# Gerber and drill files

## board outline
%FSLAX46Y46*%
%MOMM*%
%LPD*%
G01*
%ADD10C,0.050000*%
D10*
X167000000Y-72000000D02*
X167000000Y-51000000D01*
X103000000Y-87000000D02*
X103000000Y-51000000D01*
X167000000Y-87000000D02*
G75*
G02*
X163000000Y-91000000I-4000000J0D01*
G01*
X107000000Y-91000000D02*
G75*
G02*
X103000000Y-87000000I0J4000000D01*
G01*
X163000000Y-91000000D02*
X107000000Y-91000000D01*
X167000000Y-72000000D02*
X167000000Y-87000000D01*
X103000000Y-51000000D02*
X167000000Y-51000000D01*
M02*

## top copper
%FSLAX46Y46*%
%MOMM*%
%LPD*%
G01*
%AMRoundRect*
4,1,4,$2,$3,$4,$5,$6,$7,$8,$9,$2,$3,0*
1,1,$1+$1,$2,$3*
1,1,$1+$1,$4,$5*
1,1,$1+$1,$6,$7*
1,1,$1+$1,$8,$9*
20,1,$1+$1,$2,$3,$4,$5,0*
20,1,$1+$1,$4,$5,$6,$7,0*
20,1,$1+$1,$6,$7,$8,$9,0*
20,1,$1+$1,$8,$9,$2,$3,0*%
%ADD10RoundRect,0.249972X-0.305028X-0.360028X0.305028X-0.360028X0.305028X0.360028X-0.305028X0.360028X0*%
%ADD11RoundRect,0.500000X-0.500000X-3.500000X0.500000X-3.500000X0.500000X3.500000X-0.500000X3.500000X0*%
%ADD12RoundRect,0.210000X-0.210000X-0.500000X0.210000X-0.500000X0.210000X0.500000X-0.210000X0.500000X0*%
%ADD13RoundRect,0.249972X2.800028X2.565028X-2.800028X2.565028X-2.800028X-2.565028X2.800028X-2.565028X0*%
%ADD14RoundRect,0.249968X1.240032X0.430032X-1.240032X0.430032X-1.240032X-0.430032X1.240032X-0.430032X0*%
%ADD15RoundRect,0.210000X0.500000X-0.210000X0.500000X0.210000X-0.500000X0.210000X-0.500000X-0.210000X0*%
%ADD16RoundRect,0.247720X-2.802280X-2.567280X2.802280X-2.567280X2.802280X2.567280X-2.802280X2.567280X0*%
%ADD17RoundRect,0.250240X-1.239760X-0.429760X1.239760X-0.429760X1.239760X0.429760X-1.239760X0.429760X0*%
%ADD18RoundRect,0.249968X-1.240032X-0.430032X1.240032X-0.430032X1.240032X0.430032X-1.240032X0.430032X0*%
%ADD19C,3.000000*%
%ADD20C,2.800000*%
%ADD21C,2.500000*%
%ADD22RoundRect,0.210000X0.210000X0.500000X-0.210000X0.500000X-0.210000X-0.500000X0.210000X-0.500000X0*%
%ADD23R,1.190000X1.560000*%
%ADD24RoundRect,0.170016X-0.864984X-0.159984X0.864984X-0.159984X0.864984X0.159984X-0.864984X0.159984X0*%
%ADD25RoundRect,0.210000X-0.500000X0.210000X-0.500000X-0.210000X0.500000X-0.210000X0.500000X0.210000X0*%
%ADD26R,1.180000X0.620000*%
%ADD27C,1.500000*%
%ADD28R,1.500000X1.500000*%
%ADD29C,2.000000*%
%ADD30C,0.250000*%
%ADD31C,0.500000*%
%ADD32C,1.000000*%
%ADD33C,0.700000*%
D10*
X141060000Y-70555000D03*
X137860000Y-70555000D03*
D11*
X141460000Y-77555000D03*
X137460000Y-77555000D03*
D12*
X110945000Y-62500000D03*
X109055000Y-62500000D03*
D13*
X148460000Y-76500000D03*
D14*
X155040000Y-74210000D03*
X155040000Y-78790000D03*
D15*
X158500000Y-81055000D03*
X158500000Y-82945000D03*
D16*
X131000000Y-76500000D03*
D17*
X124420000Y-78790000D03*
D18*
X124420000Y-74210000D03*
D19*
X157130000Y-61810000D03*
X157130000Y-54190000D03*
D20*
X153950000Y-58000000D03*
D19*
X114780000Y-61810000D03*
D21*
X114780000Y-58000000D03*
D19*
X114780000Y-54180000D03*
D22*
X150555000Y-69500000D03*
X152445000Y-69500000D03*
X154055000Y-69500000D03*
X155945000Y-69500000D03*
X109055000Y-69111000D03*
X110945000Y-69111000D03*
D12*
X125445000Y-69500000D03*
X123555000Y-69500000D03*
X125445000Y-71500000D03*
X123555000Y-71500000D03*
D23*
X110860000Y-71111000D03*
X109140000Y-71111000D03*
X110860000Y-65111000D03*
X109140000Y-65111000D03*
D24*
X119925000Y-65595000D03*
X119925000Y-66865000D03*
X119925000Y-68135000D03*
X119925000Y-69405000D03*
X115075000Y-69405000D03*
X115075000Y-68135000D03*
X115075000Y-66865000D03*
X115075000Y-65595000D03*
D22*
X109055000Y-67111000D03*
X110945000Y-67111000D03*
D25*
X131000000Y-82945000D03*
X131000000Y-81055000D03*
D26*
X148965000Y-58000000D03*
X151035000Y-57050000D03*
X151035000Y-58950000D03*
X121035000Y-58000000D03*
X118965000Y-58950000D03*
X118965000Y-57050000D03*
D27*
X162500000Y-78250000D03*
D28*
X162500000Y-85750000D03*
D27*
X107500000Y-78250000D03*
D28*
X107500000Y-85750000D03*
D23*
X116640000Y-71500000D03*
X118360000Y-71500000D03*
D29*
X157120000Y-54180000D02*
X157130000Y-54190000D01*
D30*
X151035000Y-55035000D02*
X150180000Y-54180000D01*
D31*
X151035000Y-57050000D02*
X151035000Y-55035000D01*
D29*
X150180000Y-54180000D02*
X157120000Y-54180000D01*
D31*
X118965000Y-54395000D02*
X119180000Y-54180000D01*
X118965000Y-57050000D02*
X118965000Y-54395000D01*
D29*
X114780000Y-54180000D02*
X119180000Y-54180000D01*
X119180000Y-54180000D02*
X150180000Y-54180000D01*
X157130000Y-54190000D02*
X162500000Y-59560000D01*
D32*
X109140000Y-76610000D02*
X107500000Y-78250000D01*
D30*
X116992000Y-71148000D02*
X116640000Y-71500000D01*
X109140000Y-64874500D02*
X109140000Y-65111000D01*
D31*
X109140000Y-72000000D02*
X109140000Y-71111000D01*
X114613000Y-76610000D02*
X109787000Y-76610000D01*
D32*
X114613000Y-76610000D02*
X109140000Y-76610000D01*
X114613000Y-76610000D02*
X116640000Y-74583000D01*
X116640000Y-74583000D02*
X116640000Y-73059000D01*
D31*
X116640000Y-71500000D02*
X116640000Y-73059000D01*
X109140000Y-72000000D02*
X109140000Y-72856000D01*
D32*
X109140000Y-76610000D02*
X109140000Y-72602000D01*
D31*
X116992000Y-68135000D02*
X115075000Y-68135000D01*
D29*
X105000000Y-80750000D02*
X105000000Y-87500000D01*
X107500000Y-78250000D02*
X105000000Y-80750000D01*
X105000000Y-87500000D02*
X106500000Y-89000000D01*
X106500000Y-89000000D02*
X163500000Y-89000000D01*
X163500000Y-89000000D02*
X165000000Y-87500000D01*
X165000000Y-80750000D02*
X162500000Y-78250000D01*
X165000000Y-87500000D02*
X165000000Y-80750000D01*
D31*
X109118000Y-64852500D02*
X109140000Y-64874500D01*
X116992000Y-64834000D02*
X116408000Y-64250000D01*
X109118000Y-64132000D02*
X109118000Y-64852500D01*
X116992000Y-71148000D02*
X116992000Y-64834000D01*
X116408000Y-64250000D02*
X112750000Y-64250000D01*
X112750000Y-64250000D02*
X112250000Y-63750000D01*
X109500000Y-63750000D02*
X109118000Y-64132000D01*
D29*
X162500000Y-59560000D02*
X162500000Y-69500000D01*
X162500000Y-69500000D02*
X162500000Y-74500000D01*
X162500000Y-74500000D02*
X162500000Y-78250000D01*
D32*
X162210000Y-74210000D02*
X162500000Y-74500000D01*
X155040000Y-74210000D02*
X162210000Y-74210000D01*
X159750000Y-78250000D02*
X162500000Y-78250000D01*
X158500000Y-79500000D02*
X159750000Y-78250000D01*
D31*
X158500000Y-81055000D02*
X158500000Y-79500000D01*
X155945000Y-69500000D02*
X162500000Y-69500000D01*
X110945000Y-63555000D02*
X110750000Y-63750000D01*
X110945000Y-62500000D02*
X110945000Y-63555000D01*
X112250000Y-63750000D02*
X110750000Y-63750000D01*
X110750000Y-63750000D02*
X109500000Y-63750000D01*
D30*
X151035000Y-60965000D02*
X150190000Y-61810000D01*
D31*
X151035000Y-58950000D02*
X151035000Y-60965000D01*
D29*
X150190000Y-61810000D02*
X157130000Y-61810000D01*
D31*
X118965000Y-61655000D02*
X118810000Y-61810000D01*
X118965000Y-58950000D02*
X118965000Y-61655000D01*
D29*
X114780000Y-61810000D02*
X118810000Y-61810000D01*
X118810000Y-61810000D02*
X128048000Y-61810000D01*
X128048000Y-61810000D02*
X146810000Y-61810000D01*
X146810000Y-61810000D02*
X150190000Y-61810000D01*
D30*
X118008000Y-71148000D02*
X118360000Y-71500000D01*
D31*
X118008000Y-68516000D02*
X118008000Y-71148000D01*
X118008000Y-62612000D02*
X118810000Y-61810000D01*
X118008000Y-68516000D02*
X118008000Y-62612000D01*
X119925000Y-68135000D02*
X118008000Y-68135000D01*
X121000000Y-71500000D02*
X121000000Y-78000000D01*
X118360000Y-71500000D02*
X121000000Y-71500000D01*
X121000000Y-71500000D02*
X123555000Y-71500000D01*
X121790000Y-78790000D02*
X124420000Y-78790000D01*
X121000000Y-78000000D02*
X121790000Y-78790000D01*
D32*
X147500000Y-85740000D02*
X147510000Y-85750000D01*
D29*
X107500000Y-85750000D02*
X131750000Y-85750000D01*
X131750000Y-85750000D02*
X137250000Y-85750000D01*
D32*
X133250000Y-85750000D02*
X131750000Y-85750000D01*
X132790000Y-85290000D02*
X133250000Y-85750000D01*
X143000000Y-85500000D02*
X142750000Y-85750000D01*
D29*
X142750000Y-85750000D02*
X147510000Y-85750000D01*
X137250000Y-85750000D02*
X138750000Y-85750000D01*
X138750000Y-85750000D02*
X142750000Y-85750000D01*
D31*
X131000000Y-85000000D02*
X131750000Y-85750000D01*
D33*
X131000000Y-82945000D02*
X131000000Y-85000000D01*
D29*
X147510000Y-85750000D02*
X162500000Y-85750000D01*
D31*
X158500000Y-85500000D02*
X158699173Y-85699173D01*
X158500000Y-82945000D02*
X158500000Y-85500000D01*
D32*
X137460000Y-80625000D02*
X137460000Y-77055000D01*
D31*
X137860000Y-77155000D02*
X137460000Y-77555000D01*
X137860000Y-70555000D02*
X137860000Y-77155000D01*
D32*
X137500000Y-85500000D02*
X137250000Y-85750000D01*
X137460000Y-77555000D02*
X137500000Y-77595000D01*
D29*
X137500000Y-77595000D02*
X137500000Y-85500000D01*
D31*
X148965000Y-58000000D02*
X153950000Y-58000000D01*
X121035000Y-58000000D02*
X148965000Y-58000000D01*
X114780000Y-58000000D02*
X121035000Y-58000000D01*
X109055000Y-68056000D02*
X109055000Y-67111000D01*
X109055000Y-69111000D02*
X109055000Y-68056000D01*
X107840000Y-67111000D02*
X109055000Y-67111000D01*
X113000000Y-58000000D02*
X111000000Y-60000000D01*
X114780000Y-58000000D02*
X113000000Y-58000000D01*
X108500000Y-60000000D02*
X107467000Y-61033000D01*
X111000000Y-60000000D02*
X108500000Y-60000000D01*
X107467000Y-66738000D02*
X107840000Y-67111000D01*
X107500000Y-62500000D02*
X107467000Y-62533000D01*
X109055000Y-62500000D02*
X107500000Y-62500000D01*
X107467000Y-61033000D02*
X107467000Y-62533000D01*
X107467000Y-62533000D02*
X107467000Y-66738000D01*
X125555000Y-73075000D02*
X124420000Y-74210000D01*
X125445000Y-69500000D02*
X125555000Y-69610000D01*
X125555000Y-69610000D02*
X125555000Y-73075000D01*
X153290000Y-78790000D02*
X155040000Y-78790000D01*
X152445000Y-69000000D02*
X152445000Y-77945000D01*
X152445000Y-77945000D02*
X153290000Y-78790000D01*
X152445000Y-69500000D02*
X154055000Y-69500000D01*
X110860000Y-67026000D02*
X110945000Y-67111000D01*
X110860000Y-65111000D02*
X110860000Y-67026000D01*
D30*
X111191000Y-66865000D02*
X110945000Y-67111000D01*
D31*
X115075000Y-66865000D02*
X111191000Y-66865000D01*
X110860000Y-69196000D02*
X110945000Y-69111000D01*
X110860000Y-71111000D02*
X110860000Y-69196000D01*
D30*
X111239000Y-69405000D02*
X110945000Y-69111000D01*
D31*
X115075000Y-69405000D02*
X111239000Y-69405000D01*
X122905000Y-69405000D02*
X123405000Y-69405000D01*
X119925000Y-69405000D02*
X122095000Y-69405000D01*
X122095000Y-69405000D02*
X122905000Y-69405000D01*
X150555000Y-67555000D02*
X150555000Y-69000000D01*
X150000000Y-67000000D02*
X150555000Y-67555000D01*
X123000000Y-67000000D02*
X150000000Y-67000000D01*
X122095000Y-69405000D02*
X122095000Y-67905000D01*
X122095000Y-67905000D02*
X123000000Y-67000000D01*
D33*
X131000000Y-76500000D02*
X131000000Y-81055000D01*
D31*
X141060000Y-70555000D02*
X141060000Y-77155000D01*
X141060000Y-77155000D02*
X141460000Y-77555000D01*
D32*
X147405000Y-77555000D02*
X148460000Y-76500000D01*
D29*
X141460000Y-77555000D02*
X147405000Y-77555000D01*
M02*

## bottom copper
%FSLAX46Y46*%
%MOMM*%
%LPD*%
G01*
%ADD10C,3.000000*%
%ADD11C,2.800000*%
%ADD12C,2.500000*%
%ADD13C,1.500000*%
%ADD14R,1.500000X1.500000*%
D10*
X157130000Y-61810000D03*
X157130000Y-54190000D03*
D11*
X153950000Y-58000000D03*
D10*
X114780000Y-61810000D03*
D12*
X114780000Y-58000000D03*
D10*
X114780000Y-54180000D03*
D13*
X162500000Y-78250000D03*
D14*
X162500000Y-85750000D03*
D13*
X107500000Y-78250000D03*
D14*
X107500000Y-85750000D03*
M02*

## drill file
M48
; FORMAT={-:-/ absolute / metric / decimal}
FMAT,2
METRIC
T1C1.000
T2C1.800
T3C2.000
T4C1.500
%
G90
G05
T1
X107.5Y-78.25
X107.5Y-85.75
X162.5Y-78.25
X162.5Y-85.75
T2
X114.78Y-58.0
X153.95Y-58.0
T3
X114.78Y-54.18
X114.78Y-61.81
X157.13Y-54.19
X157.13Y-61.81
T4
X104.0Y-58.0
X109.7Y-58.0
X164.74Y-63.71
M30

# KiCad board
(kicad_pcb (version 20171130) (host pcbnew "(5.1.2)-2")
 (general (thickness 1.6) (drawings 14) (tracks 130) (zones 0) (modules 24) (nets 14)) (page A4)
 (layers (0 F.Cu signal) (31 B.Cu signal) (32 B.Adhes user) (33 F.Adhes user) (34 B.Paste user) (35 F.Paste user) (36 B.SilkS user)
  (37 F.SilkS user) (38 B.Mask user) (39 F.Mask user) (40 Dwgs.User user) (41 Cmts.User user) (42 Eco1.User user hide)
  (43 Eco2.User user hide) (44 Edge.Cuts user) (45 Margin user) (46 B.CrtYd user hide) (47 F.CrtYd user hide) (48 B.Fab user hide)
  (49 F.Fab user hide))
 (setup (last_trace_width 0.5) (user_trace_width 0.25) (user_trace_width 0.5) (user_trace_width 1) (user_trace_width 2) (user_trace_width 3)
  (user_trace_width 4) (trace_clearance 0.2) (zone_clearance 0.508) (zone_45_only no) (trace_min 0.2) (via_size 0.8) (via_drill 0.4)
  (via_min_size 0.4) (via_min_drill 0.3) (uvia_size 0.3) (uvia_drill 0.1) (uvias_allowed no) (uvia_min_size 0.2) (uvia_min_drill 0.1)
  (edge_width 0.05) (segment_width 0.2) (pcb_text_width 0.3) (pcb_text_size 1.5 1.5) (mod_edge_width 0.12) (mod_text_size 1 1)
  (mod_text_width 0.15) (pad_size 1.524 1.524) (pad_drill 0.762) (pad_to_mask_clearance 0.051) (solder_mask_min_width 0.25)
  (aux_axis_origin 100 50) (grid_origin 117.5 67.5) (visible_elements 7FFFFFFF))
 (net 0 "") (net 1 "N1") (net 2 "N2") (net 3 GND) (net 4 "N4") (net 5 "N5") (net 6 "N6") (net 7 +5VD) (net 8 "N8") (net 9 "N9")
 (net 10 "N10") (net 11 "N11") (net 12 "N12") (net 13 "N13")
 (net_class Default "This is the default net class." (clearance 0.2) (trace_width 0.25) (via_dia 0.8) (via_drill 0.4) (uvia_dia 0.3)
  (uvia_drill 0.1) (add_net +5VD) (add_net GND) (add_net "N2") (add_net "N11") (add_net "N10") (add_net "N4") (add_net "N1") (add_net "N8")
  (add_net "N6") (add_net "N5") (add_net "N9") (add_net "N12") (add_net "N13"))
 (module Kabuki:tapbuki (layer F.Cu) (at 136 58)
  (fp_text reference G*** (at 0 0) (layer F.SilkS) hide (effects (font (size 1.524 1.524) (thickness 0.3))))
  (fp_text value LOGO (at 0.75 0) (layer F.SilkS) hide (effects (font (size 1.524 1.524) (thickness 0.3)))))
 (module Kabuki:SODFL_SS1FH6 (layer F.Cu) (at 139.46 70.555)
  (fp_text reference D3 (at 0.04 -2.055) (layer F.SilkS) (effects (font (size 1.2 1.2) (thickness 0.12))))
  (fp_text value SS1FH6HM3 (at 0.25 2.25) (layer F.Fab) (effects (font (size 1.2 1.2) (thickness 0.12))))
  (pad A smd roundrect (at 1.6 0) (size 1.11 1.22) (layers F.Cu F.Paste F.Mask) (roundrect_rratio 0.2252) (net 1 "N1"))
  (pad C smd roundrect (at -1.6 0) (size 1.11 1.22) (layers F.Cu F.Paste F.Mask) (roundrect_rratio 0.2252) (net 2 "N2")))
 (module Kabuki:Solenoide (layer F.Cu) (at 137.46 77.555)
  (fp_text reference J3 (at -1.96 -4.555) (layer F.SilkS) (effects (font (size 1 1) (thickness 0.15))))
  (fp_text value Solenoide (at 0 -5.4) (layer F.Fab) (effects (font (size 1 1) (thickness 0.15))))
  (pad 2 smd roundrect (at 4 0) (size 2 8) (layers F.Cu F.Paste F.Mask) (roundrect_rratio 0.25) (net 1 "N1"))
  (pad 1 smd roundrect (at 0 0) (size 2 8) (layers F.Cu F.Paste F.Mask) (roundrect_rratio 0.25) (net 2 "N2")))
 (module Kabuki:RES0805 (layer F.Cu) (at 110 62.5)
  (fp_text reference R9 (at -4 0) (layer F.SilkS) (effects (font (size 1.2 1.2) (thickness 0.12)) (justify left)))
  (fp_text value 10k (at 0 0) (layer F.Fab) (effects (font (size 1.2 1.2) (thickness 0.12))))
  (pad 2 smd roundrect (at 0.945 0) (size 0.84 1.42) (layers F.Cu F.Paste F.Mask) (roundrect_rratio 0.25) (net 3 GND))
  (pad 1 smd roundrect (at -0.945 0) (size 0.84 1.42) (layers F.Cu F.Paste F.Mask) (roundrect_rratio 0.25) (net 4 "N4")))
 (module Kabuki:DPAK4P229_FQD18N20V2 (layer F.Cu) (at 150.97 76.5 90)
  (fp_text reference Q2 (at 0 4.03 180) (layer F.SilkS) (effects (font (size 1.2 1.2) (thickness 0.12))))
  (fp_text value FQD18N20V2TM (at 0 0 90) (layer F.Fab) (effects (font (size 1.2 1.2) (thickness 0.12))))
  (pad "" smd rect (at -1.405 -4.55 180) (size 1.44 1.92) (layers F.Paste))
  (pad "" smd rect (at -1.405 -2.51 180) (size 1.44 1.92) (layers F.Paste))
  (pad "" smd rect (at -1.405 -0.47 180) (size 1.44 1.92) (layers F.Paste))
  (pad "" smd rect (at 1.405 -4.55 180) (size 1.44 1.92) (layers F.Paste))
  (pad "" smd rect (at 1.405 -2.51 180) (size 1.44 1.92) (layers F.Paste))
  (pad "" smd rect (at 1.405 -0.47 180) (size 1.44 1.92) (layers F.Paste))
  (pad 3 smd roundrect (at 0 -2.51 180) (size 6.1 5.63) (layers F.Cu F.Mask) (roundrect_rratio 0.0444) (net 1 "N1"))
  (pad 2 smd roundrect (at 2.29 4.07 180) (size 2.98 1.36) (layers F.Cu F.Paste F.Mask) (roundrect_rratio 0.1838) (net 3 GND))
  (pad 1 smd roundrect (at -2.29 4.07 180) (size 2.98 1.36) (layers F.Cu F.Paste F.Mask) (roundrect_rratio 0.1838) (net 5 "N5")))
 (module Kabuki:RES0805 (layer F.Cu) (at 158.5 82 90)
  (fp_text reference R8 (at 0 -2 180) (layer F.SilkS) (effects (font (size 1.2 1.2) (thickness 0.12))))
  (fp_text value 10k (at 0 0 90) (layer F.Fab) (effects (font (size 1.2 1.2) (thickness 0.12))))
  (pad 2 smd roundrect (at 0.945 0 90) (size 0.84 1.42) (layers F.Cu F.Paste F.Mask) (roundrect_rratio 0.25) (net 3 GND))
  (pad 1 smd roundrect (at -0.945 0 90) (size 0.84 1.42) (layers F.Cu F.Paste F.Mask) (roundrect_rratio 0.25) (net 2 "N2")))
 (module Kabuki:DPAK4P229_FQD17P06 (layer F.Cu) (at 128.49 76.5 270)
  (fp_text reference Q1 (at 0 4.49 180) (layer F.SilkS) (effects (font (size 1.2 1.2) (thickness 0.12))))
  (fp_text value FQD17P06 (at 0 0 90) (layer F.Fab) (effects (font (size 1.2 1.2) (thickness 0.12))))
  (pad "" smd rect (at -1.405 -4.55) (size 1.44 1.92) (layers F.Paste))
  (pad "" smd rect (at -1.405 -2.51) (size 1.44 1.92) (layers F.Paste))
  (pad "" smd rect (at -1.405 -0.47) (size 1.44 1.92) (layers F.Paste))
  (pad "" smd rect (at 1.405 -4.55) (size 1.44 1.92) (layers F.Paste))
  (pad "" smd rect (at 1.405 -2.51) (size 1.44 1.92) (layers F.Paste))
  (pad "" smd rect (at 1.405 -0.47) (size 1.44 1.92) (layers F.Paste))
  (pad 4 smd roundrect (at 0 -2.51) (size 6.1 5.63) (layers F.Cu F.Mask) (roundrect_rratio 0.044) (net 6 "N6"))
  (pad 3 smd roundrect (at 2.29 4.07) (size 2.98 1.36) (layers F.Cu F.Paste F.Mask) (roundrect_rratio 0.184) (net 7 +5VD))
  (pad 1 smd roundrect (at -2.29 4.07) (size 2.98 1.36) (layers F.Cu F.Paste F.Mask) (roundrect_rratio 0.1838) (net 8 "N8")))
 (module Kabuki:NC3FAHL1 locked (layer B.Cu) (at 173 58 90)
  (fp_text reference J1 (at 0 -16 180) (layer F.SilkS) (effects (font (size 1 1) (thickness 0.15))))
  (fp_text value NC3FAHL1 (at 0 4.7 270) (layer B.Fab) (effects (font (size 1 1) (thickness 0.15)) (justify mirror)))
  (pad 3 thru_hole circle (at -3.81 -15.87 90) (size 3 3) (drill 2) (layers *.Cu *.Mask) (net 7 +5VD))
  (pad "" np_thru_hole circle (at -5.71 -8.26 90) (size 1.5 1.5) (drill 1.5) (layers *.Cu *.Mask))
  (pad 1 thru_hole circle (at 3.81 -15.87 90) (size 3 3) (drill 2) (layers *.Cu *.Mask) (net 3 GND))
  (pad 2 thru_hole circle (at 0 -19.05 90) (size 2.8 2.8) (drill 1.8) (layers *.Cu *.Mask) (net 4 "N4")))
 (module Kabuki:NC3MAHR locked (layer B.Cu) (at 97 58 270)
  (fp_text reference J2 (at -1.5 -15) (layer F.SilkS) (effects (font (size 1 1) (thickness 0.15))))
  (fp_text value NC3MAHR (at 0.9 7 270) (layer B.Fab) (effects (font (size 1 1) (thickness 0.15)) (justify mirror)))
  (pad "" np_thru_hole circle (at 0 -7 270) (size 1.5 1.5) (drill 1.5) (layers *.Cu *.Mask))
  (pad "" np_thru_hole circle (at 0 -12.7 270) (size 1.5 1.5) (drill 1.5) (layers *.Cu *.Mask))
  (pad 3 thru_hole circle (at 3.81 -17.78 270) (size 3 3) (drill 2) (layers *.Cu *.Mask) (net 7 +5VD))
  (pad 2 thru_hole circle (at 0 -17.78 270) (size 2.5 2.5) (drill 1.8) (layers *.Cu *.Mask) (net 4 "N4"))
  (pad 1 thru_hole circle (at -3.82 -17.78 270) (size 3 3) (drill 2) (layers *.Cu *.Mask) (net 3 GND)))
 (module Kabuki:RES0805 (layer F.Cu) (at 151.5 69.5 180)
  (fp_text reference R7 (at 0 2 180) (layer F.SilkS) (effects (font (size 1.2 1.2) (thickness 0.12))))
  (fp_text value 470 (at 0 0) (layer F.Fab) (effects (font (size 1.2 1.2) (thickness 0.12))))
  (pad 2 smd roundrect (at 0.945 0 180) (size 0.84 1.42) (layers F.Cu F.Paste F.Mask) (roundrect_rratio 0.25) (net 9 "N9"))
  (pad 1 smd roundrect (at -0.945 0 180) (size 0.84 1.42) (layers F.Cu F.Paste F.Mask) (roundrect_rratio 0.25) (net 5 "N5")))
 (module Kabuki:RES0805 (layer F.Cu) (at 155 69.5 180)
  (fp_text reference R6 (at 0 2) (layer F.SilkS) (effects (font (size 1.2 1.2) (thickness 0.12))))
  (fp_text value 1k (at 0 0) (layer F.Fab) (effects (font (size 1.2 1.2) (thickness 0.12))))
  (pad 2 smd roundrect (at 0.945 0 180) (size 0.84 1.42) (layers F.Cu F.Paste F.Mask) (roundrect_rratio 0.25) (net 5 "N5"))
  (pad 1 smd roundrect (at -0.945 0 180) (size 0.84 1.42) (layers F.Cu F.Paste F.Mask) (roundrect_rratio 0.25) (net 3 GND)))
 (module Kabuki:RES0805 (layer F.Cu) (at 110 69.111 180)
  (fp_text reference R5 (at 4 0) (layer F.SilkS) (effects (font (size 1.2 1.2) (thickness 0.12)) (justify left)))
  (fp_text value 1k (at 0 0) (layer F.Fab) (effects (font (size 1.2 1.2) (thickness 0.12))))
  (pad 2 smd roundrect (at 0.945 0 180) (size 0.84 1.42) (layers F.Cu F.Paste F.Mask) (roundrect_rratio 0.25) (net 4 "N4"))
  (pad 1 smd roundrect (at -0.945 0 180) (size 0.84 1.42) (layers F.Cu F.Paste F.Mask) (roundrect_rratio 0.25) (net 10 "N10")))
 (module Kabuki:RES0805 (layer F.Cu) (at 124.5 69.5)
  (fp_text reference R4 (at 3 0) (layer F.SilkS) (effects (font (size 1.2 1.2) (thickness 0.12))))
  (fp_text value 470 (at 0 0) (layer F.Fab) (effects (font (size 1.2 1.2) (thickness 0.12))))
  (pad 2 smd roundrect (at 0.945 0) (size 0.84 1.42) (layers F.Cu F.Paste F.Mask) (roundrect_rratio 0.25) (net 8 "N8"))
  (pad 1 smd roundrect (at -0.945 0) (size 0.84 1.42) (layers F.Cu F.Paste F.Mask) (roundrect_rratio 0.25) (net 9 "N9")))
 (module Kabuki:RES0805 (layer F.Cu) (at 124.5 71.5)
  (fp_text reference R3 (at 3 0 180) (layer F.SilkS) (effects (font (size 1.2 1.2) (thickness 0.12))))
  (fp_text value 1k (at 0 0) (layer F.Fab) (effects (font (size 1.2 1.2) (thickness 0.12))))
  (pad 2 smd roundrect (at 0.945 0) (size 0.84 1.42) (layers F.Cu F.Paste F.Mask) (roundrect_rratio 0.25) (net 8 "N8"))
  (pad 1 smd roundrect (at -0.945 0) (size 0.84 1.42) (layers F.Cu F.Paste F.Mask) (roundrect_rratio 0.25) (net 7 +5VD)))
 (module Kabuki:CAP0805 (layer F.Cu) (at 110 71.111)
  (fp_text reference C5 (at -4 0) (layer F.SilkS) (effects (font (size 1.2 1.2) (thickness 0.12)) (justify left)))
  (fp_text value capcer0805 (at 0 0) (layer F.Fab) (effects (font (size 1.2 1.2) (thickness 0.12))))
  (pad 2 smd rect (at 0.86 0) (size 1.19 1.56) (layers F.Cu F.Paste F.Mask) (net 10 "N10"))
  (pad 1 smd rect (at -0.86 0) (size 1.19 1.56) (layers F.Cu F.Paste F.Mask) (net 3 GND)))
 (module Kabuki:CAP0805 (layer F.Cu) (at 110 65.111)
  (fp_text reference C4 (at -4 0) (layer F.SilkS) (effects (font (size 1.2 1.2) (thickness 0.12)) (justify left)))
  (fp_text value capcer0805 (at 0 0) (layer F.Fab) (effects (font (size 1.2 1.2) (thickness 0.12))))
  (pad 2 smd rect (at 0.86 0) (size 1.19 1.56) (layers F.Cu F.Paste F.Mask) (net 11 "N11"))
  (pad 1 smd rect (at -0.86 0) (size 1.19 1.56) (layers F.Cu F.Paste F.Mask) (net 3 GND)))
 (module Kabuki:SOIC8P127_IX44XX (layer F.Cu) (at 117.5 67.5 270)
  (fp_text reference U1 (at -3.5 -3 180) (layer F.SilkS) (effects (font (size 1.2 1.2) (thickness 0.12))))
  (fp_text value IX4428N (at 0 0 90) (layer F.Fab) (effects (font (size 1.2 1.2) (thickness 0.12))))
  (pad 8 smd roundrect (at -1.905 -2.425) (size 2.07 0.66) (layers F.Cu F.Paste F.Mask) (roundrect_rratio 0.2576) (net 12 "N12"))
  (pad 7 smd roundrect (at -0.635 -2.425) (size 2.07 0.66) (layers F.Cu F.Paste F.Mask) (roundrect_rratio 0.2576) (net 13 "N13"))
  (pad 6 smd roundrect (at 0.635 -2.425) (size 2.07 0.66) (layers F.Cu F.Paste F.Mask) (roundrect_rratio 0.2576) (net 7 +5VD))
  (pad 5 smd roundrect (at 1.905 -2.425) (size 2.07 0.66) (layers F.Cu F.Paste F.Mask) (roundrect_rratio 0.2576) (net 9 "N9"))
  (pad 4 smd roundrect (at 1.905 2.425) (size 2.07 0.66) (layers F.Cu F.Paste F.Mask) (roundrect_rratio 0.2576) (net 10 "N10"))
  (pad 3 smd roundrect (at 0.635 2.425) (size 2.07 0.66) (layers F.Cu F.Paste F.Mask) (roundrect_rratio 0.2576) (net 3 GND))
  (pad 2 smd roundrect (at -0.635 2.425) (size 2.07 0.66) (layers F.Cu F.Paste F.Mask) (roundrect_rratio 0.2576) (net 11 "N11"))
  (pad 1 smd roundrect (at -1.905 2.425) (size 2.07 0.66) (layers F.Cu F.Paste F.Mask) (roundrect_rratio 0.2576) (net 12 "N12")))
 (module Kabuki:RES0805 (layer F.Cu) (at 110 67.111 180)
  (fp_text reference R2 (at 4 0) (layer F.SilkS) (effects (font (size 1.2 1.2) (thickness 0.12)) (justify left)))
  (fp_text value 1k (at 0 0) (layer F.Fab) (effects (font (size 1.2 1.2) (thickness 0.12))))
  (pad 2 smd roundrect (at 0.945 0 180) (size 0.84 1.42) (layers F.Cu F.Paste F.Mask) (roundrect_rratio 0.25) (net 4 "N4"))
  (pad 1 smd roundrect (at -0.945 0 180) (size 0.84 1.42) (layers F.Cu F.Paste F.Mask) (roundrect_rratio 0.25) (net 11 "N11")))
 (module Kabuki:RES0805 (layer F.Cu) (at 131 82 270)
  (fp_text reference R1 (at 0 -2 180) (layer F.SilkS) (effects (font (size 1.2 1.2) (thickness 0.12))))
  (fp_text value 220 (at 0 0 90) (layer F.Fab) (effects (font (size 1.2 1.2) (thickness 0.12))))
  (pad 2 smd roundrect (at 0.945 0 270) (size 0.84 1.42) (layers F.Cu F.Paste F.Mask) (roundrect_rratio 0.25) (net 2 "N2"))
  (pad 1 smd roundrect (at -0.945 0 270) (size 0.84 1.42) (layers F.Cu F.Paste F.Mask) (roundrect_rratio 0.25) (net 6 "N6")))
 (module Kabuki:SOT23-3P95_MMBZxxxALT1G (layer F.Cu) (at 150 58 90)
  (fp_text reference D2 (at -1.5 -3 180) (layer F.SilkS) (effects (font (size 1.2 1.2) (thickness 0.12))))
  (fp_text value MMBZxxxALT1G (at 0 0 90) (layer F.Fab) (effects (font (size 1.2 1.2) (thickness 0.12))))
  (pad 3 smd rect (at 0 -1.035 180) (size 1.18 0.62) (layers F.Cu F.Paste F.Mask) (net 4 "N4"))
  (pad 2 smd rect (at 0.95 1.035 180) (size 1.18 0.62) (layers F.Cu F.Paste F.Mask) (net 3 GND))
  (pad 1 smd rect (at -0.95 1.035 180) (size 1.18 0.62) (layers F.Cu F.Paste F.Mask) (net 7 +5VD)))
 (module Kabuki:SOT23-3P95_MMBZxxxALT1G (layer F.Cu) (at 120 58 270)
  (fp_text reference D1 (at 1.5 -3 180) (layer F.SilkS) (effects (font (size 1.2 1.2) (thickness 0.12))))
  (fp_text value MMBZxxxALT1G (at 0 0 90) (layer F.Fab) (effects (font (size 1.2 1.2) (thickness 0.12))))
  (pad 3 smd rect (at 0 -1.035) (size 1.18 0.62) (layers F.Cu F.Paste F.Mask) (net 4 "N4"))
  (pad 2 smd rect (at 0.95 1.035) (size 1.18 0.62) (layers F.Cu F.Paste F.Mask) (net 7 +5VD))
  (pad 1 smd rect (at -0.95 1.035) (size 1.18 0.62) (layers F.Cu F.Paste F.Mask) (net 3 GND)))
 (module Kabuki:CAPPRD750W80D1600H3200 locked (layer B.Cu) (at 162.5 82 90)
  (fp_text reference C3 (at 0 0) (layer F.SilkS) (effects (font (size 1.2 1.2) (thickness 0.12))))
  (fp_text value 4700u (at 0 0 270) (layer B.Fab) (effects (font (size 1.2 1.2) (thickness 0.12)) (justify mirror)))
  (pad 2 thru_hole circle (at 3.75 0 90) (size 1.5 1.5) (drill 1) (layers *.Cu *.Mask) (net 3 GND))
  (pad 1 thru_hole rect (at -3.75 0 90) (size 1.5 1.5) (drill 1) (layers *.Cu *.Mask) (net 2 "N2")))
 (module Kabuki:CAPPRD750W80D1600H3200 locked (layer B.Cu) (at 107.5 82 90)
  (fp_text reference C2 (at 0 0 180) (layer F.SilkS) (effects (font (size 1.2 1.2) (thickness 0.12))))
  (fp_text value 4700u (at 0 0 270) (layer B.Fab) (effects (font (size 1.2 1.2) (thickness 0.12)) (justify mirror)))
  (pad 2 thru_hole circle (at 3.75 0 90) (size 1.5 1.5) (drill 1) (layers *.Cu *.Mask) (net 3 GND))
  (pad 1 thru_hole rect (at -3.75 0 90) (size 1.5 1.5) (drill 1) (layers *.Cu *.Mask) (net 2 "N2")))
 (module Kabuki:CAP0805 (layer F.Cu) (at 117.5 71.5 180)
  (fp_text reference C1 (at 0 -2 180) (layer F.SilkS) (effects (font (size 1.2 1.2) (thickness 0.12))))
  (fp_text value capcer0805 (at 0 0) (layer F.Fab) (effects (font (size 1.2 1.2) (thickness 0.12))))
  (pad 2 smd rect (at 0.86 0 180) (size 1.19 1.56) (layers F.Cu F.Paste F.Mask) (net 3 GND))
  (pad 1 smd rect (at -0.86 0 180) (size 1.19 1.56) (layers F.Cu F.Paste F.Mask) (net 7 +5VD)))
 (gr_line (start 167 72) (end 167 51) (layer Edge.Cuts) (width 0.05))
 (gr_line (start 103 87) (end 103 51) (layer Edge.Cuts) (width 0.05))
 (gr_arc (start 163 87) (end 163 91) (angle -90) (layer Edge.Cuts) (width 0.05))
 (gr_arc (start 107 87) (end 103 87) (angle -90) (layer Edge.Cuts) (width 0.05))
 (gr_line (start 163 91) (end 107 91) (layer Edge.Cuts) (width 0.05))
 (gr_line (start 167 72) (end 167 87) (layer Edge.Cuts) (width 0.05))
 (gr_line (start 103 51) (end 167 51) (layer Edge.Cuts) (width 0.05))
 (segment (start 157.12 54.18) (end 157.13 54.19) (width 2) (layer F.Cu) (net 3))
 (segment (start 151.035 55.035) (end 150.18 54.18) (width 0.25) (layer F.Cu) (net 3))
 (segment (start 151.035 57.05) (end 151.035 55.035) (width 0.5) (layer F.Cu) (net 3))
 (segment (start 150.18 54.18) (end 157.12 54.18) (width 2) (layer F.Cu) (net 3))
 (segment (start 118.965 54.395) (end 119.18 54.18) (width 0.5) (layer F.Cu) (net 3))
 (segment (start 118.965 57.05) (end 118.965 54.395) (width 0.5) (layer F.Cu) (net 3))
 (segment (start 114.78 54.18) (end 119.18 54.18) (width 2) (layer F.Cu) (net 3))
 (segment (start 119.18 54.18) (end 150.18 54.18) (width 2) (layer F.Cu) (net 3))
 (segment (start 157.13 54.19) (end 162.5 59.56) (width 2) (layer F.Cu) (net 3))
 (segment (start 109.14 76.61) (end 107.5 78.25) (width 1) (layer F.Cu) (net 3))
 (segment (start 116.992 71.148) (end 116.64 71.5) (width 0.25) (layer F.Cu) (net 3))
 (segment (start 109.14 64.8745) (end 109.14 65.111) (width 0.25) (layer F.Cu) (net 3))
 (segment (start 109.14 72) (end 109.14 71.111) (width 0.5) (layer F.Cu) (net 3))
 (segment (start 114.613 76.61) (end 109.787 76.61) (width 0.5) (layer F.Cu) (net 3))
 (segment (start 114.613 76.61) (end 109.14 76.61) (width 1) (layer F.Cu) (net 3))
 (segment (start 114.613 76.61) (end 116.64 74.583) (width 1) (layer F.Cu) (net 3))
 (segment (start 116.64 74.583) (end 116.64 73.059) (width 1) (layer F.Cu) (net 3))
 (segment (start 116.64 71.5) (end 116.64 73.059) (width 0.5) (layer F.Cu) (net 3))
 (segment (start 109.14 72) (end 109.14 72.856) (width 0.5) (layer F.Cu) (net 3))
 (segment (start 109.14 76.61) (end 109.14 72.602) (width 1) (layer F.Cu) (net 3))
 (segment (start 116.992 68.135) (end 115.075 68.135) (width 0.5) (layer F.Cu) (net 3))
 (segment (start 105 80.75) (end 105 87.5) (width 2) (layer F.Cu) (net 3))
 (segment (start 107.5 78.25) (end 105 80.75) (width 2) (layer F.Cu) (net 3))
 (segment (start 105 87.5) (end 106.5 89) (width 2) (layer F.Cu) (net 3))
 (segment (start 106.5 89) (end 163.5 89) (width 2) (layer F.Cu) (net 3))
 (segment (start 163.5 89) (end 165 87.5) (width 2) (layer F.Cu) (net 3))
 (segment (start 165 80.75) (end 162.5 78.25) (width 2) (layer F.Cu) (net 3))
 (segment (start 165 87.5) (end 165 80.75) (width 2) (layer F.Cu) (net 3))
 (segment (start 109.118 64.8525) (end 109.14 64.8745) (width 0.5) (layer F.Cu) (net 3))
 (segment (start 116.992 64.834) (end 116.408 64.25) (width 0.5) (layer F.Cu) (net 3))
 (segment (start 109.118 64.132) (end 109.118 64.8525) (width 0.5) (layer F.Cu) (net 3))
 (segment (start 116.992 71.148) (end 116.992 64.834) (width 0.5) (layer F.Cu) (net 3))
 (segment (start 116.408 64.25) (end 112.75 64.25) (width 0.5) (layer F.Cu) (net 3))
 (segment (start 112.75 64.25) (end 112.25 63.75) (width 0.5) (layer F.Cu) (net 3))
 (segment (start 109.5 63.75) (end 109.118 64.132) (width 0.5) (layer F.Cu) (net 3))
 (segment (start 162.5 59.56) (end 162.5 69.5) (width 2) (layer F.Cu) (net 3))
 (segment (start 162.5 69.5) (end 162.5 74.5) (width 2) (layer F.Cu) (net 3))
 (segment (start 162.5 74.5) (end 162.5 78.25) (width 2) (layer F.Cu) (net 3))
 (segment (start 162.21 74.21) (end 162.5 74.5) (width 1) (layer F.Cu) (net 3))
 (segment (start 155.04 74.21) (end 162.21 74.21) (width 1) (layer F.Cu) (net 3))
 (segment (start 159.75 78.25) (end 162.5 78.25) (width 1) (layer F.Cu) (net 3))
 (segment (start 158.5 79.5) (end 159.75 78.25) (width 1) (layer F.Cu) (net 3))
 (segment (start 158.5 81.055) (end 158.5 79.5) (width 0.5) (layer F.Cu) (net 3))
 (segment (start 155.945 69.5) (end 162.5 69.5) (width 0.5) (layer F.Cu) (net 3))
 (segment (start 110.945 63.555) (end 110.75 63.75) (width 0.5) (layer F.Cu) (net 3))
 (segment (start 110.945 62.5) (end 110.945 63.555) (width 0.5) (layer F.Cu) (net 3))
 (segment (start 112.25 63.75) (end 110.75 63.75) (width 0.5) (layer F.Cu) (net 3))
 (segment (start 110.75 63.75) (end 109.5 63.75) (width 0.5) (layer F.Cu) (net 3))
 (segment (start 151.035 60.965) (end 150.19 61.81) (width 0.25) (layer F.Cu) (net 7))
 (segment (start 151.035 58.95) (end 151.035 60.965) (width 0.5) (layer F.Cu) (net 7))
 (segment (start 150.19 61.81) (end 157.13 61.81) (width 2) (layer F.Cu) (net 7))
 (segment (start 118.965 61.655) (end 118.81 61.81) (width 0.5) (layer F.Cu) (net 7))
 (segment (start 118.965 58.95) (end 118.965 61.655) (width 0.5) (layer F.Cu) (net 7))
 (segment (start 114.78 61.81) (end 118.81 61.81) (width 2) (layer F.Cu) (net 7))
 (segment (start 118.81 61.81) (end 128.048 61.81) (width 2) (layer F.Cu) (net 7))
 (segment (start 128.048 61.81) (end 146.81 61.81) (width 2) (layer F.Cu) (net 7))
 (segment (start 146.81 61.81) (end 150.19 61.81) (width 2) (layer F.Cu) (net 7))
 (segment (start 118.008 71.148) (end 118.36 71.5) (width 0.25) (layer F.Cu) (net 7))
 (segment (start 118.008 68.516) (end 118.008 71.148) (width 0.5) (layer F.Cu) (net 7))
 (segment (start 118.008 62.612) (end 118.81 61.81) (width 0.5) (layer F.Cu) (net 7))
 (segment (start 118.008 68.516) (end 118.008 62.612) (width 0.5) (layer F.Cu) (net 7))
 (segment (start 119.925 68.135) (end 118.008 68.135) (width 0.5) (layer F.Cu) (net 7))
 (segment (start 121 71.5) (end 121 78) (width 0.5) (layer F.Cu) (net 7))
 (segment (start 118.36 71.5) (end 121 71.5) (width 0.5) (layer F.Cu) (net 7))
 (segment (start 121 71.5) (end 123.555 71.5) (width 0.5) (layer F.Cu) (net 7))
 (segment (start 121.79 78.79) (end 124.42 78.79) (width 0.5) (layer F.Cu) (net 7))
 (segment (start 121 78) (end 121.79 78.79) (width 0.5) (layer F.Cu) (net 7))
 (segment (start 147.5 85.74) (end 147.51 85.75) (width 1) (layer F.Cu) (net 2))
 (segment (start 107.5 85.75) (end 131.75 85.75) (width 2) (layer F.Cu) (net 2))
 (segment (start 131.75 85.75) (end 137.25 85.75) (width 2) (layer F.Cu) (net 2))
 (segment (start 133.25 85.75) (end 131.75 85.75) (width 1) (layer F.Cu) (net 2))
 (segment (start 132.79 85.29) (end 133.25 85.75) (width 1) (layer F.Cu) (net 2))
 (segment (start 143 85.5) (end 142.75 85.75) (width 1) (layer F.Cu) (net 2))
 (segment (start 142.75 85.75) (end 147.51 85.75) (width 2) (layer F.Cu) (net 2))
 (segment (start 137.25 85.75) (end 138.75 85.75) (width 2) (layer F.Cu) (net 2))
 (segment (start 138.75 85.75) (end 142.75 85.75) (width 2) (layer F.Cu) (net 2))
 (segment (start 131 85) (end 131.75 85.75) (width 0.5) (layer F.Cu) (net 2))
 (segment (start 131 82.945) (end 131 85) (width 0.7) (layer F.Cu) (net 2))
 (segment (start 147.51 85.75) (end 162.5 85.75) (width 2) (layer F.Cu) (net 2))
 (segment (start 158.5 85.5) (end 158.699173 85.699173) (width 0.5) (layer F.Cu) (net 2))
 (segment (start 158.5 82.945) (end 158.5 85.5) (width 0.5) (layer F.Cu) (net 2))
 (segment (start 137.46 80.625) (end 137.46 77.055) (width 1) (layer F.Cu) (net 2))
 (segment (start 137.86 77.155) (end 137.46 77.555) (width 0.5) (layer F.Cu) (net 2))
 (segment (start 137.86 70.555) (end 137.86 77.155) (width 0.5) (layer F.Cu) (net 2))
 (segment (start 137.5 85.5) (end 137.25 85.75) (width 1) (layer F.Cu) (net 2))
 (segment (start 137.46 77.555) (end 137.5 77.595) (width 1) (layer F.Cu) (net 2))
 (segment (start 137.5 77.595) (end 137.5 85.5) (width 2) (layer F.Cu) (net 2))
 (segment (start 148.965 58) (end 153.95 58) (width 0.5) (layer F.Cu) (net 4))
 (segment (start 121.035 58) (end 148.965 58) (width 0.5) (layer F.Cu) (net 4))
 (segment (start 114.78 58) (end 121.035 58) (width 0.5) (layer F.Cu) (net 4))
 (segment (start 109.055 68.056) (end 109.055 67.111) (width 0.5) (layer F.Cu) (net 4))
 (segment (start 109.055 69.111) (end 109.055 68.056) (width 0.5) (layer F.Cu) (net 4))
 (segment (start 107.84 67.111) (end 109.055 67.111) (width 0.5) (layer F.Cu) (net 4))
 (segment (start 113 58) (end 111 60) (width 0.5) (layer F.Cu) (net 4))
 (segment (start 114.78 58) (end 113 58) (width 0.5) (layer F.Cu) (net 4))
 (segment (start 108.5 60) (end 107.467 61.033) (width 0.5) (layer F.Cu) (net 4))
 (segment (start 111 60) (end 108.5 60) (width 0.5) (layer F.Cu) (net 4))
 (segment (start 107.467 66.738) (end 107.84 67.111) (width 0.5) (layer F.Cu) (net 4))
 (segment (start 107.5 62.5) (end 107.467 62.533) (width 0.5) (layer F.Cu) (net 4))
 (segment (start 109.055 62.5) (end 107.5 62.5) (width 0.5) (layer F.Cu) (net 4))
 (segment (start 107.467 61.033) (end 107.467 62.533) (width 0.5) (layer F.Cu) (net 4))
 (segment (start 107.467 62.533) (end 107.467 66.738) (width 0.5) (layer F.Cu) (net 4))
 (segment (start 125.555 73.075) (end 124.42 74.21) (width 0.5) (layer F.Cu) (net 8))
 (segment (start 125.445 69.5) (end 125.555 69.61) (width 0.5) (layer F.Cu) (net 8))
 (segment (start 125.555 69.61) (end 125.555 73.075) (width 0.5) (layer F.Cu) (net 8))
 (segment (start 153.29 78.79) (end 155.04 78.79) (width 0.5) (layer F.Cu) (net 5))
 (segment (start 152.445 69) (end 152.445 77.945) (width 0.5) (layer F.Cu) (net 5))
 (segment (start 152.445 77.945) (end 153.29 78.79) (width 0.5) (layer F.Cu) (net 5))
 (segment (start 152.445 69.5) (end 154.055 69.5) (width 0.5) (layer F.Cu) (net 5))
 (segment (start 110.86 67.026) (end 110.945 67.111) (width 0.5) (layer F.Cu) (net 11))
 (segment (start 110.86 65.111) (end 110.86 67.026) (width 0.5) (layer F.Cu) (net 11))
 (segment (start 111.191 66.865) (end 110.945 67.111) (width 0.25) (layer F.Cu) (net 11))
 (segment (start 115.075 66.865) (end 111.191 66.865) (width 0.5) (layer F.Cu) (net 11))
 (segment (start 110.86 69.196) (end 110.945 69.111) (width 0.5) (layer F.Cu) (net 10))
 (segment (start 110.86 71.111) (end 110.86 69.196) (width 0.5) (layer F.Cu) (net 10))
 (segment (start 111.239 69.405) (end 110.945 69.111) (width 0.25) (layer F.Cu) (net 10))
 (segment (start 115.075 69.405) (end 111.239 69.405) (width 0.5) (layer F.Cu) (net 10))
 (segment (start 122.905 69.405) (end 123.405 69.405) (width 0.5) (layer F.Cu) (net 9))
 (segment (start 119.925 69.405) (end 122.095 69.405) (width 0.5) (layer F.Cu) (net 9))
 (segment (start 122.095 69.405) (end 122.905 69.405) (width 0.5) (layer F.Cu) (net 9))
 (segment (start 150.555 67.555) (end 150.555 69) (width 0.5) (layer F.Cu) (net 9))
 (segment (start 150 67) (end 150.555 67.555) (width 0.5) (layer F.Cu) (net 9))
 (segment (start 123 67) (end 150 67) (width 0.5) (layer F.Cu) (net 9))
 (segment (start 122.095 69.405) (end 122.095 67.905) (width 0.5) (layer F.Cu) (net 9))
 (segment (start 122.095 67.905) (end 123 67) (width 0.5) (layer F.Cu) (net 9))
 (segment (start 131 76.5) (end 131 81.055) (width 0.7) (layer F.Cu) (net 6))
 (segment (start 141.06 70.555) (end 141.06 77.155) (width 0.5) (layer F.Cu) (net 1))
 (segment (start 141.06 77.155) (end 141.46 77.555) (width 0.5) (layer F.Cu) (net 1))
 (segment (start 147.405 77.555) (end 148.46 76.5) (width 1) (layer F.Cu) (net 1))
 (segment (start 141.46 77.555) (end 147.405 77.555) (width 2) (layer F.Cu) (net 1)))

